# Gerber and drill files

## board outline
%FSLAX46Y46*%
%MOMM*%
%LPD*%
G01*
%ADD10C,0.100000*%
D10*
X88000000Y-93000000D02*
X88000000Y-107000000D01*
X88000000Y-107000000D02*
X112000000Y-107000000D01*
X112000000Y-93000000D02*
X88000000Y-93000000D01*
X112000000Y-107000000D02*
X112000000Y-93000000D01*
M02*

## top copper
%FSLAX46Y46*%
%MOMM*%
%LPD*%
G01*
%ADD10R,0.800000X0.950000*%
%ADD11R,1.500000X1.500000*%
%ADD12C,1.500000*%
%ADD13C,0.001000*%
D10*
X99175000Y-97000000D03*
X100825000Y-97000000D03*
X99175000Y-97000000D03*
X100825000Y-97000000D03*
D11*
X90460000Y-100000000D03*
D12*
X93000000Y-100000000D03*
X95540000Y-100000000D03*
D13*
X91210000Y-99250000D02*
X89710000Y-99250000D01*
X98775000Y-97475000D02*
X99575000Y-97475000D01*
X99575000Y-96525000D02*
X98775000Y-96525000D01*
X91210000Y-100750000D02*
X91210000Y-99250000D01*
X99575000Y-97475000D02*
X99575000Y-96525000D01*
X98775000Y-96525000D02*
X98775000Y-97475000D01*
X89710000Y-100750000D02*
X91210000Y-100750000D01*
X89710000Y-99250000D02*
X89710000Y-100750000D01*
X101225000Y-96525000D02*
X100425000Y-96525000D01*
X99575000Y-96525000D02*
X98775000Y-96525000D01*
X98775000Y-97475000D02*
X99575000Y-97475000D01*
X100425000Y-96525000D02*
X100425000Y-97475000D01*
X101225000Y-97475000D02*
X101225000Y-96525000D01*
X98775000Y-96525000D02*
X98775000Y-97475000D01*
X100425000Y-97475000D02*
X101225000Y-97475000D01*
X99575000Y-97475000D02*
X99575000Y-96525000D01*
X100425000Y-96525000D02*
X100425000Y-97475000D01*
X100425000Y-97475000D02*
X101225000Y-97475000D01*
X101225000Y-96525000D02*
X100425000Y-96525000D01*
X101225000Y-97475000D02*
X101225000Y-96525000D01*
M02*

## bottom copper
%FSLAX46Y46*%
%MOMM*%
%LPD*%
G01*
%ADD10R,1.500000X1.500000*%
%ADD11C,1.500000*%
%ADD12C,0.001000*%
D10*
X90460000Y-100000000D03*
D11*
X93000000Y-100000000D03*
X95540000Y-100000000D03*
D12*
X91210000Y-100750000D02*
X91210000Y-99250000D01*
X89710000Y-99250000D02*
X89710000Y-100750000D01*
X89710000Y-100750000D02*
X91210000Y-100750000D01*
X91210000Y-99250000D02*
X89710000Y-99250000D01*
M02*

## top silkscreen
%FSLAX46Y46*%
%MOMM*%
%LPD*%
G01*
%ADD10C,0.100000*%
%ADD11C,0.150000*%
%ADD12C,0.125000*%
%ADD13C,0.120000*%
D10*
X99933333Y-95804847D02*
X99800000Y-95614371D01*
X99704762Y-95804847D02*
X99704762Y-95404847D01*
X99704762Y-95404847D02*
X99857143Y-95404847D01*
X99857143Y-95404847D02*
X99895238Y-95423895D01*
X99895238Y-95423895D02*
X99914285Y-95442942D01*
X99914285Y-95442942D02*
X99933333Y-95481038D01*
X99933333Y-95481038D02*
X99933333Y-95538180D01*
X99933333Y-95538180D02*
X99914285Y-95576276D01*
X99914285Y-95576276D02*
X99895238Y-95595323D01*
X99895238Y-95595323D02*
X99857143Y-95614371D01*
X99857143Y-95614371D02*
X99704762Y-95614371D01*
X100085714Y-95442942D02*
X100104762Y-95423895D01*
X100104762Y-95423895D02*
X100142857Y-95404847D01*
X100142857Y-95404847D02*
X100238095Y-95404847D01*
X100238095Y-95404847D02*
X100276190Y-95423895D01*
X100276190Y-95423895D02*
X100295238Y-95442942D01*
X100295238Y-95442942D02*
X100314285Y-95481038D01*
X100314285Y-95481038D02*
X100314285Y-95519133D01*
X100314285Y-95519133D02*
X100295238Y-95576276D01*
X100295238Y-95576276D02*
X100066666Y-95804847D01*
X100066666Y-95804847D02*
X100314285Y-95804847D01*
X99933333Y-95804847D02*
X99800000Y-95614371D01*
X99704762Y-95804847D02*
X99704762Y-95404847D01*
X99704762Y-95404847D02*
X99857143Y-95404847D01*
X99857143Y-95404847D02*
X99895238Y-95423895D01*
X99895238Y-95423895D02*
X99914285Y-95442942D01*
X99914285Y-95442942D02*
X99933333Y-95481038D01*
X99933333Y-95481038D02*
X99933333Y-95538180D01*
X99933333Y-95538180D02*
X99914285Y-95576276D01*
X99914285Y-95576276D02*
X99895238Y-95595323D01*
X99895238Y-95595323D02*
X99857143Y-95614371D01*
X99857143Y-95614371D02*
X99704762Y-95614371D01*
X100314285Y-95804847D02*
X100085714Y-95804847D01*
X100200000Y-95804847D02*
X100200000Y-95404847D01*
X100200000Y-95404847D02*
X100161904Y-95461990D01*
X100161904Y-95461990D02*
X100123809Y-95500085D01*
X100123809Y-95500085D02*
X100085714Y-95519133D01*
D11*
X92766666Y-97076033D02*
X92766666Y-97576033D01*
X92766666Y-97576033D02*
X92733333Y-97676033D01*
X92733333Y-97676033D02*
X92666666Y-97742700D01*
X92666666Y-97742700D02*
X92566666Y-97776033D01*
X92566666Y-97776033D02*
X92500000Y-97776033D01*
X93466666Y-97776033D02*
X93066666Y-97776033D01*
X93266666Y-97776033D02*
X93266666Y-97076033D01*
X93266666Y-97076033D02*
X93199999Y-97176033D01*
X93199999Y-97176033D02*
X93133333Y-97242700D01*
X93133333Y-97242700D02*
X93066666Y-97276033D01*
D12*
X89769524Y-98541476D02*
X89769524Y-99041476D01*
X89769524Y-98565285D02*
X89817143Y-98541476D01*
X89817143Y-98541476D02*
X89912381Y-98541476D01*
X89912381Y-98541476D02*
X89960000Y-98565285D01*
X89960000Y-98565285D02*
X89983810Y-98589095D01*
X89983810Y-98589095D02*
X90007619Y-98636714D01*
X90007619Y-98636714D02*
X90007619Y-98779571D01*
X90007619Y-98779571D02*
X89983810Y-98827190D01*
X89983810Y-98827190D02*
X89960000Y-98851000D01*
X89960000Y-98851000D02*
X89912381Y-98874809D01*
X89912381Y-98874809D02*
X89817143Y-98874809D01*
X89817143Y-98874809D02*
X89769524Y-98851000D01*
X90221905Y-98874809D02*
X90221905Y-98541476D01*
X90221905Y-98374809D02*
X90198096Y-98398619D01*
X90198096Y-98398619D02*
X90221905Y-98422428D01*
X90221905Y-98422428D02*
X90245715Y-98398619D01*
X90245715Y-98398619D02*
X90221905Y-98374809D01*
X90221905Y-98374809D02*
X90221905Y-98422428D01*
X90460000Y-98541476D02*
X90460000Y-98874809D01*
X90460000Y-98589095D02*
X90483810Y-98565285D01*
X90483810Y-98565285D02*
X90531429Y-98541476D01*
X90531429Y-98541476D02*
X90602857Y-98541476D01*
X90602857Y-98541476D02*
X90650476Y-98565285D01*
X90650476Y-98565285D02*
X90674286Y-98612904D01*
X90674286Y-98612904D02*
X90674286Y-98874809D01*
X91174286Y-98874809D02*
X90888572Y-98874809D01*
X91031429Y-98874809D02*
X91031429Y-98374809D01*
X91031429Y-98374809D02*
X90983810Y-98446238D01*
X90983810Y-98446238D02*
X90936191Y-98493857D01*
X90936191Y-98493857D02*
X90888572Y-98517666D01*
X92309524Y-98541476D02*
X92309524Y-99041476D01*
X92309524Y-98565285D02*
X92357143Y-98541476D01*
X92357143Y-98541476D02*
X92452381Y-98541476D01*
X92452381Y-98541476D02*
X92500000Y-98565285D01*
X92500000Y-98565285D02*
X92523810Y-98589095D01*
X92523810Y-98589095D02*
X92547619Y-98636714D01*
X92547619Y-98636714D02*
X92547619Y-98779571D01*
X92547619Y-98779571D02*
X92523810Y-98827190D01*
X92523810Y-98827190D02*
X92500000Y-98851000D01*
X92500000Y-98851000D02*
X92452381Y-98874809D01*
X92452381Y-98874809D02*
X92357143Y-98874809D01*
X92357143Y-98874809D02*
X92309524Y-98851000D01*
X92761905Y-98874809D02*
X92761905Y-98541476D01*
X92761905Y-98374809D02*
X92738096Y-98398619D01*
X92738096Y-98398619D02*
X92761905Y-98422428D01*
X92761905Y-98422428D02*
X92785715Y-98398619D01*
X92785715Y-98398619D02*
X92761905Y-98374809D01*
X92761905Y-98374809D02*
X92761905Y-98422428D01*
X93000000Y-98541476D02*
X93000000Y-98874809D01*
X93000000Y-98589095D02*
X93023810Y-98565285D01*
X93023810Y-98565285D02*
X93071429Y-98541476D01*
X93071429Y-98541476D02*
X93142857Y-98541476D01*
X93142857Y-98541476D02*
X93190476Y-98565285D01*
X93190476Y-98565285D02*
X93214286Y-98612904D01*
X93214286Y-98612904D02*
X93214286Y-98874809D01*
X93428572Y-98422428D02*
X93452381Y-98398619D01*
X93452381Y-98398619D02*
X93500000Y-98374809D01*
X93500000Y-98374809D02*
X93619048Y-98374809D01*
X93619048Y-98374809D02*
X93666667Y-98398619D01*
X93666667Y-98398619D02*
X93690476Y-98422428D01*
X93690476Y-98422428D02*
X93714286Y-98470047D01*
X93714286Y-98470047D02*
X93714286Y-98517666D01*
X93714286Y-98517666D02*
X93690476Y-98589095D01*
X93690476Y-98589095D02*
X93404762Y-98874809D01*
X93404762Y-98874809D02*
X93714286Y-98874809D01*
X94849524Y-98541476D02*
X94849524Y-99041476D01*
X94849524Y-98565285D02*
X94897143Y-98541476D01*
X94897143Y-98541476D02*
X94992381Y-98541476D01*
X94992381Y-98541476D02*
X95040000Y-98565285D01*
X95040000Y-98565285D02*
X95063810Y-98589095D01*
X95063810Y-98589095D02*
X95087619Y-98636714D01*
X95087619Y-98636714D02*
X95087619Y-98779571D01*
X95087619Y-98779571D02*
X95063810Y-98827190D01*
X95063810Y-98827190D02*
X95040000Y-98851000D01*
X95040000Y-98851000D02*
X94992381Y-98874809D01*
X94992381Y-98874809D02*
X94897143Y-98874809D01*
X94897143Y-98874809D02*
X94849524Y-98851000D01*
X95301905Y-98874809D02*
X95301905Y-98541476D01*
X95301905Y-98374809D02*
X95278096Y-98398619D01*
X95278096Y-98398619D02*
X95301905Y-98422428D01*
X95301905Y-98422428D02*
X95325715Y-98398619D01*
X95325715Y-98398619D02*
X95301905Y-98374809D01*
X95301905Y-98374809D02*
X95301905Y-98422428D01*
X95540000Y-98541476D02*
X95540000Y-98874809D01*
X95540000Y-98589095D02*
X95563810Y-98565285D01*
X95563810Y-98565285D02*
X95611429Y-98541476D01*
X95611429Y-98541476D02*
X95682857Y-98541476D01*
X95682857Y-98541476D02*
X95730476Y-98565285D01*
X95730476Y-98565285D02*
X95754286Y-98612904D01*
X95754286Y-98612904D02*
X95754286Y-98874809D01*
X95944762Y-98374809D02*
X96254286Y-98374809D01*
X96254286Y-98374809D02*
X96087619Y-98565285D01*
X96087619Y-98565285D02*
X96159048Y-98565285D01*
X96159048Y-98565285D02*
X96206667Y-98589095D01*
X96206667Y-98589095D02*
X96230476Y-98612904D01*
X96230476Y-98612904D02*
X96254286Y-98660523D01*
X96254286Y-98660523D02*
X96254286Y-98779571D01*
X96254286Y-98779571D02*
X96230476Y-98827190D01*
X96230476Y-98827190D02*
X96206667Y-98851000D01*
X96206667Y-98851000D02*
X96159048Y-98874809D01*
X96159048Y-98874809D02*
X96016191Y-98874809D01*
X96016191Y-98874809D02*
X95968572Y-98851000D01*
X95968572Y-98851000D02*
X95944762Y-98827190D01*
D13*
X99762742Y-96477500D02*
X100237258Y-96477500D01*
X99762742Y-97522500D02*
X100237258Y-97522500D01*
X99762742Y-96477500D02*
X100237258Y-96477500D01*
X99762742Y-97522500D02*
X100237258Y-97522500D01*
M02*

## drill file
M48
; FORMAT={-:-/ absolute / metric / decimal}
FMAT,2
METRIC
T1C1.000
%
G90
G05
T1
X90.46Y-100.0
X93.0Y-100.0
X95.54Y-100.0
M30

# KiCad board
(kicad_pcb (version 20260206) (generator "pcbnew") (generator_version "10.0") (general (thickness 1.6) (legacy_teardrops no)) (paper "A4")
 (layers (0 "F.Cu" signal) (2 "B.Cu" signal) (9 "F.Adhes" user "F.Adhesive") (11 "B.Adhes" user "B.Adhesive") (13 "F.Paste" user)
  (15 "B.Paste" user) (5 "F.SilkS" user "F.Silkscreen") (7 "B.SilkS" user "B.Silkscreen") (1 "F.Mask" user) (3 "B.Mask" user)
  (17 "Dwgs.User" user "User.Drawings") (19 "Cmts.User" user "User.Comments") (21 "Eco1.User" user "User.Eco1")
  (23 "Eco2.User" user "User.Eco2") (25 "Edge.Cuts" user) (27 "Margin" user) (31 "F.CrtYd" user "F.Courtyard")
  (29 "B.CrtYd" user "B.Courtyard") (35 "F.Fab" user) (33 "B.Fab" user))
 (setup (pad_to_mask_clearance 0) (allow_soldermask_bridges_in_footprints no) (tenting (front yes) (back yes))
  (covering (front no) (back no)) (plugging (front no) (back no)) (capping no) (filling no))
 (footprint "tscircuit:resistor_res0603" (layer "F.Cu") (at 100 97)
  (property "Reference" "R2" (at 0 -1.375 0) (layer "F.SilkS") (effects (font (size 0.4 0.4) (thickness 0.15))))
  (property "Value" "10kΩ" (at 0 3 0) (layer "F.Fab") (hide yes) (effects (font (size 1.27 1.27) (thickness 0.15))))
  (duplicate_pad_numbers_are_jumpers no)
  (fp_line (start -0.237258 -0.5225) (end 0.237258 -0.5225) (stroke (width 0.12) (type default)) (layer "F.SilkS"))
  (fp_line (start -0.237258 0.5225) (end 0.237258 0.5225) (stroke (width 0.12) (type default)) (layer "F.SilkS"))
  (pad "" smd rect (at -0.825 0) (size 0.56 0.665) (layers "F.Paste"))
  (pad "" smd rect (at 0.825 0) (size 0.56 0.665) (layers "F.Paste"))
  (pad "1" smd rect (at -0.825 0) (size 0.8 0.95) (layers "F.Cu" "F.Mask") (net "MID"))
  (pad "2" smd rect (at 0.825 0) (size 0.8 0.95) (layers "F.Cu" "F.Mask") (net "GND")))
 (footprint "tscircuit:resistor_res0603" (layer "F.Cu") (at 100 97)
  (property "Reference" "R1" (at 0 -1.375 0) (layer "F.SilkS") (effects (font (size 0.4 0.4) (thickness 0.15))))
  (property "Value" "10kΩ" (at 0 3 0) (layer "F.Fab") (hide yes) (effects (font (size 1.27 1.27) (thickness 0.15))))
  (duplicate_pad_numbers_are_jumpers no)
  (fp_line (start -0.237258 -0.5225) (end 0.237258 -0.5225) (stroke (width 0.12) (type default)) (layer "F.SilkS"))
  (fp_line (start -0.237258 0.5225) (end 0.237258 0.5225) (stroke (width 0.12) (type default)) (layer "F.SilkS"))
  (pad "" smd rect (at -0.825 0) (size 0.56 0.665) (layers "F.Paste"))
  (pad "" smd rect (at 0.825 0) (size 0.56 0.665) (layers "F.Paste"))
  (pad "1" smd rect (at -0.825 0) (size 0.8 0.95) (layers "F.Cu" "F.Mask") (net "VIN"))
  (pad "2" smd rect (at 0.825 0) (size 0.8 0.95) (layers "F.Cu" "F.Mask") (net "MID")))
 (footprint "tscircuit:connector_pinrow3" (layer "F.Cu") (at 93 100)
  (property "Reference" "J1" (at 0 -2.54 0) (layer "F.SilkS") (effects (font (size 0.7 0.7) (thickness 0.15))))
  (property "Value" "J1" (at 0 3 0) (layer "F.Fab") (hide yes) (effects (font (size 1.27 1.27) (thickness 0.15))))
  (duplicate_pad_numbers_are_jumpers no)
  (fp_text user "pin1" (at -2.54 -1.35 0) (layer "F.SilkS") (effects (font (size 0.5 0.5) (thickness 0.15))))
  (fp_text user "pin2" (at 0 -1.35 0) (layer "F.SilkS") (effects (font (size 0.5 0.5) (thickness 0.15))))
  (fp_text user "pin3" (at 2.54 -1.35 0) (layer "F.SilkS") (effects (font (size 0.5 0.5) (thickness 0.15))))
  (pad "1" thru_hole rect (at -2.54 0) (size 1.5 1.5) (drill 1) (layers "*.Cu" "*.Mask") (remove_unused_layers no) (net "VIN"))
  (pad "2" thru_hole circle (at 0 0) (size 1.5 1.5) (drill 1) (layers "*.Cu" "*.Mask") (remove_unused_layers no) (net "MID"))
  (pad "3" thru_hole circle (at 2.54 0) (size 1.5 1.5) (drill 1) (layers "*.Cu" "*.Mask") (remove_unused_layers no) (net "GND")))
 (gr_line (start 88 93) (end 88 107) (stroke (width 0.1) (type solid)) (layer "Edge.Cuts"))
 (gr_line (start 88 107) (end 112 107) (stroke (width 0.1) (type solid)) (layer "Edge.Cuts"))
 (gr_line (start 112 93) (end 88 93) (stroke (width 0.1) (type solid)) (layer "Edge.Cuts"))
 (gr_line (start 112 107) (end 112 93) (stroke (width 0.1) (type solid)) (layer "Edge.Cuts"))
 (segment (start 91.21 99.25) (end 89.71 99.25) (width 0.001) (layer "F.Cu") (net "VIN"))
 (segment (start 98.775 97.475) (end 99.575 97.475) (width 0.001) (layer "F.Cu") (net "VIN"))
 (segment (start 99.575 96.525) (end 98.775 96.525) (width 0.001) (layer "F.Cu") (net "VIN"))
 (segment (start 91.21 100.75) (end 91.21 99.25) (width 0.001) (layer "F.Cu") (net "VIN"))
 (segment (start 99.575 97.475) (end 99.575 96.525) (width 0.001) (layer "F.Cu") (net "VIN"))
 (segment (start 98.775 96.525) (end 98.775 97.475) (width 0.001) (layer "F.Cu") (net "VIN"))
 (segment (start 89.71 100.75) (end 91.21 100.75) (width 0.001) (layer "F.Cu") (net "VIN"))
 (segment (start 89.71 99.25) (end 89.71 100.75) (width 0.001) (layer "F.Cu") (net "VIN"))
 (segment (start 91.21 100.75) (end 91.21 99.25) (width 0.001) (layer "B.Cu") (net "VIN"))
 (segment (start 89.71 99.25) (end 89.71 100.75) (width 0.001) (layer "B.Cu") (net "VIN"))
 (segment (start 89.71 100.75) (end 91.21 100.75) (width 0.001) (layer "B.Cu") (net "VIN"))
 (segment (start 91.21 99.25) (end 89.71 99.25) (width 0.001) (layer "B.Cu") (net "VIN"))
 (segment (start 101.225 96.525) (end 100.425 96.525) (width 0.001) (layer "F.Cu") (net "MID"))
 (segment (start 99.575 96.525) (end 98.775 96.525) (width 0.001) (layer "F.Cu") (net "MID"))
 (segment (start 98.775 97.475) (end 99.575 97.475) (width 0.001) (layer "F.Cu") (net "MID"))
 (segment (start 100.425 96.525) (end 100.425 97.475) (width 0.001) (layer "F.Cu") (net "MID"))
 (segment (start 101.225 97.475) (end 101.225 96.525) (width 0.001) (layer "F.Cu") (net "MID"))
 (segment (start 98.775 96.525) (end 98.775 97.475) (width 0.001) (layer "F.Cu") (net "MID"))
 (segment (start 100.425 97.475) (end 101.225 97.475) (width 0.001) (layer "F.Cu") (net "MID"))
 (segment (start 99.575 97.475) (end 99.575 96.525) (width 0.001) (layer "F.Cu") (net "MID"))
 (segment (start 100.425 96.525) (end 100.425 97.475) (width 0.001) (layer "F.Cu") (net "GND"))
 (segment (start 100.425 97.475) (end 101.225 97.475) (width 0.001) (layer "F.Cu") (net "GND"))
 (segment (start 101.225 96.525) (end 100.425 96.525) (width 0.001) (layer "F.Cu") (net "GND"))
 (segment (start 101.225 97.475) (end 101.225 96.525) (width 0.001) (layer "F.Cu") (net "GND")))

